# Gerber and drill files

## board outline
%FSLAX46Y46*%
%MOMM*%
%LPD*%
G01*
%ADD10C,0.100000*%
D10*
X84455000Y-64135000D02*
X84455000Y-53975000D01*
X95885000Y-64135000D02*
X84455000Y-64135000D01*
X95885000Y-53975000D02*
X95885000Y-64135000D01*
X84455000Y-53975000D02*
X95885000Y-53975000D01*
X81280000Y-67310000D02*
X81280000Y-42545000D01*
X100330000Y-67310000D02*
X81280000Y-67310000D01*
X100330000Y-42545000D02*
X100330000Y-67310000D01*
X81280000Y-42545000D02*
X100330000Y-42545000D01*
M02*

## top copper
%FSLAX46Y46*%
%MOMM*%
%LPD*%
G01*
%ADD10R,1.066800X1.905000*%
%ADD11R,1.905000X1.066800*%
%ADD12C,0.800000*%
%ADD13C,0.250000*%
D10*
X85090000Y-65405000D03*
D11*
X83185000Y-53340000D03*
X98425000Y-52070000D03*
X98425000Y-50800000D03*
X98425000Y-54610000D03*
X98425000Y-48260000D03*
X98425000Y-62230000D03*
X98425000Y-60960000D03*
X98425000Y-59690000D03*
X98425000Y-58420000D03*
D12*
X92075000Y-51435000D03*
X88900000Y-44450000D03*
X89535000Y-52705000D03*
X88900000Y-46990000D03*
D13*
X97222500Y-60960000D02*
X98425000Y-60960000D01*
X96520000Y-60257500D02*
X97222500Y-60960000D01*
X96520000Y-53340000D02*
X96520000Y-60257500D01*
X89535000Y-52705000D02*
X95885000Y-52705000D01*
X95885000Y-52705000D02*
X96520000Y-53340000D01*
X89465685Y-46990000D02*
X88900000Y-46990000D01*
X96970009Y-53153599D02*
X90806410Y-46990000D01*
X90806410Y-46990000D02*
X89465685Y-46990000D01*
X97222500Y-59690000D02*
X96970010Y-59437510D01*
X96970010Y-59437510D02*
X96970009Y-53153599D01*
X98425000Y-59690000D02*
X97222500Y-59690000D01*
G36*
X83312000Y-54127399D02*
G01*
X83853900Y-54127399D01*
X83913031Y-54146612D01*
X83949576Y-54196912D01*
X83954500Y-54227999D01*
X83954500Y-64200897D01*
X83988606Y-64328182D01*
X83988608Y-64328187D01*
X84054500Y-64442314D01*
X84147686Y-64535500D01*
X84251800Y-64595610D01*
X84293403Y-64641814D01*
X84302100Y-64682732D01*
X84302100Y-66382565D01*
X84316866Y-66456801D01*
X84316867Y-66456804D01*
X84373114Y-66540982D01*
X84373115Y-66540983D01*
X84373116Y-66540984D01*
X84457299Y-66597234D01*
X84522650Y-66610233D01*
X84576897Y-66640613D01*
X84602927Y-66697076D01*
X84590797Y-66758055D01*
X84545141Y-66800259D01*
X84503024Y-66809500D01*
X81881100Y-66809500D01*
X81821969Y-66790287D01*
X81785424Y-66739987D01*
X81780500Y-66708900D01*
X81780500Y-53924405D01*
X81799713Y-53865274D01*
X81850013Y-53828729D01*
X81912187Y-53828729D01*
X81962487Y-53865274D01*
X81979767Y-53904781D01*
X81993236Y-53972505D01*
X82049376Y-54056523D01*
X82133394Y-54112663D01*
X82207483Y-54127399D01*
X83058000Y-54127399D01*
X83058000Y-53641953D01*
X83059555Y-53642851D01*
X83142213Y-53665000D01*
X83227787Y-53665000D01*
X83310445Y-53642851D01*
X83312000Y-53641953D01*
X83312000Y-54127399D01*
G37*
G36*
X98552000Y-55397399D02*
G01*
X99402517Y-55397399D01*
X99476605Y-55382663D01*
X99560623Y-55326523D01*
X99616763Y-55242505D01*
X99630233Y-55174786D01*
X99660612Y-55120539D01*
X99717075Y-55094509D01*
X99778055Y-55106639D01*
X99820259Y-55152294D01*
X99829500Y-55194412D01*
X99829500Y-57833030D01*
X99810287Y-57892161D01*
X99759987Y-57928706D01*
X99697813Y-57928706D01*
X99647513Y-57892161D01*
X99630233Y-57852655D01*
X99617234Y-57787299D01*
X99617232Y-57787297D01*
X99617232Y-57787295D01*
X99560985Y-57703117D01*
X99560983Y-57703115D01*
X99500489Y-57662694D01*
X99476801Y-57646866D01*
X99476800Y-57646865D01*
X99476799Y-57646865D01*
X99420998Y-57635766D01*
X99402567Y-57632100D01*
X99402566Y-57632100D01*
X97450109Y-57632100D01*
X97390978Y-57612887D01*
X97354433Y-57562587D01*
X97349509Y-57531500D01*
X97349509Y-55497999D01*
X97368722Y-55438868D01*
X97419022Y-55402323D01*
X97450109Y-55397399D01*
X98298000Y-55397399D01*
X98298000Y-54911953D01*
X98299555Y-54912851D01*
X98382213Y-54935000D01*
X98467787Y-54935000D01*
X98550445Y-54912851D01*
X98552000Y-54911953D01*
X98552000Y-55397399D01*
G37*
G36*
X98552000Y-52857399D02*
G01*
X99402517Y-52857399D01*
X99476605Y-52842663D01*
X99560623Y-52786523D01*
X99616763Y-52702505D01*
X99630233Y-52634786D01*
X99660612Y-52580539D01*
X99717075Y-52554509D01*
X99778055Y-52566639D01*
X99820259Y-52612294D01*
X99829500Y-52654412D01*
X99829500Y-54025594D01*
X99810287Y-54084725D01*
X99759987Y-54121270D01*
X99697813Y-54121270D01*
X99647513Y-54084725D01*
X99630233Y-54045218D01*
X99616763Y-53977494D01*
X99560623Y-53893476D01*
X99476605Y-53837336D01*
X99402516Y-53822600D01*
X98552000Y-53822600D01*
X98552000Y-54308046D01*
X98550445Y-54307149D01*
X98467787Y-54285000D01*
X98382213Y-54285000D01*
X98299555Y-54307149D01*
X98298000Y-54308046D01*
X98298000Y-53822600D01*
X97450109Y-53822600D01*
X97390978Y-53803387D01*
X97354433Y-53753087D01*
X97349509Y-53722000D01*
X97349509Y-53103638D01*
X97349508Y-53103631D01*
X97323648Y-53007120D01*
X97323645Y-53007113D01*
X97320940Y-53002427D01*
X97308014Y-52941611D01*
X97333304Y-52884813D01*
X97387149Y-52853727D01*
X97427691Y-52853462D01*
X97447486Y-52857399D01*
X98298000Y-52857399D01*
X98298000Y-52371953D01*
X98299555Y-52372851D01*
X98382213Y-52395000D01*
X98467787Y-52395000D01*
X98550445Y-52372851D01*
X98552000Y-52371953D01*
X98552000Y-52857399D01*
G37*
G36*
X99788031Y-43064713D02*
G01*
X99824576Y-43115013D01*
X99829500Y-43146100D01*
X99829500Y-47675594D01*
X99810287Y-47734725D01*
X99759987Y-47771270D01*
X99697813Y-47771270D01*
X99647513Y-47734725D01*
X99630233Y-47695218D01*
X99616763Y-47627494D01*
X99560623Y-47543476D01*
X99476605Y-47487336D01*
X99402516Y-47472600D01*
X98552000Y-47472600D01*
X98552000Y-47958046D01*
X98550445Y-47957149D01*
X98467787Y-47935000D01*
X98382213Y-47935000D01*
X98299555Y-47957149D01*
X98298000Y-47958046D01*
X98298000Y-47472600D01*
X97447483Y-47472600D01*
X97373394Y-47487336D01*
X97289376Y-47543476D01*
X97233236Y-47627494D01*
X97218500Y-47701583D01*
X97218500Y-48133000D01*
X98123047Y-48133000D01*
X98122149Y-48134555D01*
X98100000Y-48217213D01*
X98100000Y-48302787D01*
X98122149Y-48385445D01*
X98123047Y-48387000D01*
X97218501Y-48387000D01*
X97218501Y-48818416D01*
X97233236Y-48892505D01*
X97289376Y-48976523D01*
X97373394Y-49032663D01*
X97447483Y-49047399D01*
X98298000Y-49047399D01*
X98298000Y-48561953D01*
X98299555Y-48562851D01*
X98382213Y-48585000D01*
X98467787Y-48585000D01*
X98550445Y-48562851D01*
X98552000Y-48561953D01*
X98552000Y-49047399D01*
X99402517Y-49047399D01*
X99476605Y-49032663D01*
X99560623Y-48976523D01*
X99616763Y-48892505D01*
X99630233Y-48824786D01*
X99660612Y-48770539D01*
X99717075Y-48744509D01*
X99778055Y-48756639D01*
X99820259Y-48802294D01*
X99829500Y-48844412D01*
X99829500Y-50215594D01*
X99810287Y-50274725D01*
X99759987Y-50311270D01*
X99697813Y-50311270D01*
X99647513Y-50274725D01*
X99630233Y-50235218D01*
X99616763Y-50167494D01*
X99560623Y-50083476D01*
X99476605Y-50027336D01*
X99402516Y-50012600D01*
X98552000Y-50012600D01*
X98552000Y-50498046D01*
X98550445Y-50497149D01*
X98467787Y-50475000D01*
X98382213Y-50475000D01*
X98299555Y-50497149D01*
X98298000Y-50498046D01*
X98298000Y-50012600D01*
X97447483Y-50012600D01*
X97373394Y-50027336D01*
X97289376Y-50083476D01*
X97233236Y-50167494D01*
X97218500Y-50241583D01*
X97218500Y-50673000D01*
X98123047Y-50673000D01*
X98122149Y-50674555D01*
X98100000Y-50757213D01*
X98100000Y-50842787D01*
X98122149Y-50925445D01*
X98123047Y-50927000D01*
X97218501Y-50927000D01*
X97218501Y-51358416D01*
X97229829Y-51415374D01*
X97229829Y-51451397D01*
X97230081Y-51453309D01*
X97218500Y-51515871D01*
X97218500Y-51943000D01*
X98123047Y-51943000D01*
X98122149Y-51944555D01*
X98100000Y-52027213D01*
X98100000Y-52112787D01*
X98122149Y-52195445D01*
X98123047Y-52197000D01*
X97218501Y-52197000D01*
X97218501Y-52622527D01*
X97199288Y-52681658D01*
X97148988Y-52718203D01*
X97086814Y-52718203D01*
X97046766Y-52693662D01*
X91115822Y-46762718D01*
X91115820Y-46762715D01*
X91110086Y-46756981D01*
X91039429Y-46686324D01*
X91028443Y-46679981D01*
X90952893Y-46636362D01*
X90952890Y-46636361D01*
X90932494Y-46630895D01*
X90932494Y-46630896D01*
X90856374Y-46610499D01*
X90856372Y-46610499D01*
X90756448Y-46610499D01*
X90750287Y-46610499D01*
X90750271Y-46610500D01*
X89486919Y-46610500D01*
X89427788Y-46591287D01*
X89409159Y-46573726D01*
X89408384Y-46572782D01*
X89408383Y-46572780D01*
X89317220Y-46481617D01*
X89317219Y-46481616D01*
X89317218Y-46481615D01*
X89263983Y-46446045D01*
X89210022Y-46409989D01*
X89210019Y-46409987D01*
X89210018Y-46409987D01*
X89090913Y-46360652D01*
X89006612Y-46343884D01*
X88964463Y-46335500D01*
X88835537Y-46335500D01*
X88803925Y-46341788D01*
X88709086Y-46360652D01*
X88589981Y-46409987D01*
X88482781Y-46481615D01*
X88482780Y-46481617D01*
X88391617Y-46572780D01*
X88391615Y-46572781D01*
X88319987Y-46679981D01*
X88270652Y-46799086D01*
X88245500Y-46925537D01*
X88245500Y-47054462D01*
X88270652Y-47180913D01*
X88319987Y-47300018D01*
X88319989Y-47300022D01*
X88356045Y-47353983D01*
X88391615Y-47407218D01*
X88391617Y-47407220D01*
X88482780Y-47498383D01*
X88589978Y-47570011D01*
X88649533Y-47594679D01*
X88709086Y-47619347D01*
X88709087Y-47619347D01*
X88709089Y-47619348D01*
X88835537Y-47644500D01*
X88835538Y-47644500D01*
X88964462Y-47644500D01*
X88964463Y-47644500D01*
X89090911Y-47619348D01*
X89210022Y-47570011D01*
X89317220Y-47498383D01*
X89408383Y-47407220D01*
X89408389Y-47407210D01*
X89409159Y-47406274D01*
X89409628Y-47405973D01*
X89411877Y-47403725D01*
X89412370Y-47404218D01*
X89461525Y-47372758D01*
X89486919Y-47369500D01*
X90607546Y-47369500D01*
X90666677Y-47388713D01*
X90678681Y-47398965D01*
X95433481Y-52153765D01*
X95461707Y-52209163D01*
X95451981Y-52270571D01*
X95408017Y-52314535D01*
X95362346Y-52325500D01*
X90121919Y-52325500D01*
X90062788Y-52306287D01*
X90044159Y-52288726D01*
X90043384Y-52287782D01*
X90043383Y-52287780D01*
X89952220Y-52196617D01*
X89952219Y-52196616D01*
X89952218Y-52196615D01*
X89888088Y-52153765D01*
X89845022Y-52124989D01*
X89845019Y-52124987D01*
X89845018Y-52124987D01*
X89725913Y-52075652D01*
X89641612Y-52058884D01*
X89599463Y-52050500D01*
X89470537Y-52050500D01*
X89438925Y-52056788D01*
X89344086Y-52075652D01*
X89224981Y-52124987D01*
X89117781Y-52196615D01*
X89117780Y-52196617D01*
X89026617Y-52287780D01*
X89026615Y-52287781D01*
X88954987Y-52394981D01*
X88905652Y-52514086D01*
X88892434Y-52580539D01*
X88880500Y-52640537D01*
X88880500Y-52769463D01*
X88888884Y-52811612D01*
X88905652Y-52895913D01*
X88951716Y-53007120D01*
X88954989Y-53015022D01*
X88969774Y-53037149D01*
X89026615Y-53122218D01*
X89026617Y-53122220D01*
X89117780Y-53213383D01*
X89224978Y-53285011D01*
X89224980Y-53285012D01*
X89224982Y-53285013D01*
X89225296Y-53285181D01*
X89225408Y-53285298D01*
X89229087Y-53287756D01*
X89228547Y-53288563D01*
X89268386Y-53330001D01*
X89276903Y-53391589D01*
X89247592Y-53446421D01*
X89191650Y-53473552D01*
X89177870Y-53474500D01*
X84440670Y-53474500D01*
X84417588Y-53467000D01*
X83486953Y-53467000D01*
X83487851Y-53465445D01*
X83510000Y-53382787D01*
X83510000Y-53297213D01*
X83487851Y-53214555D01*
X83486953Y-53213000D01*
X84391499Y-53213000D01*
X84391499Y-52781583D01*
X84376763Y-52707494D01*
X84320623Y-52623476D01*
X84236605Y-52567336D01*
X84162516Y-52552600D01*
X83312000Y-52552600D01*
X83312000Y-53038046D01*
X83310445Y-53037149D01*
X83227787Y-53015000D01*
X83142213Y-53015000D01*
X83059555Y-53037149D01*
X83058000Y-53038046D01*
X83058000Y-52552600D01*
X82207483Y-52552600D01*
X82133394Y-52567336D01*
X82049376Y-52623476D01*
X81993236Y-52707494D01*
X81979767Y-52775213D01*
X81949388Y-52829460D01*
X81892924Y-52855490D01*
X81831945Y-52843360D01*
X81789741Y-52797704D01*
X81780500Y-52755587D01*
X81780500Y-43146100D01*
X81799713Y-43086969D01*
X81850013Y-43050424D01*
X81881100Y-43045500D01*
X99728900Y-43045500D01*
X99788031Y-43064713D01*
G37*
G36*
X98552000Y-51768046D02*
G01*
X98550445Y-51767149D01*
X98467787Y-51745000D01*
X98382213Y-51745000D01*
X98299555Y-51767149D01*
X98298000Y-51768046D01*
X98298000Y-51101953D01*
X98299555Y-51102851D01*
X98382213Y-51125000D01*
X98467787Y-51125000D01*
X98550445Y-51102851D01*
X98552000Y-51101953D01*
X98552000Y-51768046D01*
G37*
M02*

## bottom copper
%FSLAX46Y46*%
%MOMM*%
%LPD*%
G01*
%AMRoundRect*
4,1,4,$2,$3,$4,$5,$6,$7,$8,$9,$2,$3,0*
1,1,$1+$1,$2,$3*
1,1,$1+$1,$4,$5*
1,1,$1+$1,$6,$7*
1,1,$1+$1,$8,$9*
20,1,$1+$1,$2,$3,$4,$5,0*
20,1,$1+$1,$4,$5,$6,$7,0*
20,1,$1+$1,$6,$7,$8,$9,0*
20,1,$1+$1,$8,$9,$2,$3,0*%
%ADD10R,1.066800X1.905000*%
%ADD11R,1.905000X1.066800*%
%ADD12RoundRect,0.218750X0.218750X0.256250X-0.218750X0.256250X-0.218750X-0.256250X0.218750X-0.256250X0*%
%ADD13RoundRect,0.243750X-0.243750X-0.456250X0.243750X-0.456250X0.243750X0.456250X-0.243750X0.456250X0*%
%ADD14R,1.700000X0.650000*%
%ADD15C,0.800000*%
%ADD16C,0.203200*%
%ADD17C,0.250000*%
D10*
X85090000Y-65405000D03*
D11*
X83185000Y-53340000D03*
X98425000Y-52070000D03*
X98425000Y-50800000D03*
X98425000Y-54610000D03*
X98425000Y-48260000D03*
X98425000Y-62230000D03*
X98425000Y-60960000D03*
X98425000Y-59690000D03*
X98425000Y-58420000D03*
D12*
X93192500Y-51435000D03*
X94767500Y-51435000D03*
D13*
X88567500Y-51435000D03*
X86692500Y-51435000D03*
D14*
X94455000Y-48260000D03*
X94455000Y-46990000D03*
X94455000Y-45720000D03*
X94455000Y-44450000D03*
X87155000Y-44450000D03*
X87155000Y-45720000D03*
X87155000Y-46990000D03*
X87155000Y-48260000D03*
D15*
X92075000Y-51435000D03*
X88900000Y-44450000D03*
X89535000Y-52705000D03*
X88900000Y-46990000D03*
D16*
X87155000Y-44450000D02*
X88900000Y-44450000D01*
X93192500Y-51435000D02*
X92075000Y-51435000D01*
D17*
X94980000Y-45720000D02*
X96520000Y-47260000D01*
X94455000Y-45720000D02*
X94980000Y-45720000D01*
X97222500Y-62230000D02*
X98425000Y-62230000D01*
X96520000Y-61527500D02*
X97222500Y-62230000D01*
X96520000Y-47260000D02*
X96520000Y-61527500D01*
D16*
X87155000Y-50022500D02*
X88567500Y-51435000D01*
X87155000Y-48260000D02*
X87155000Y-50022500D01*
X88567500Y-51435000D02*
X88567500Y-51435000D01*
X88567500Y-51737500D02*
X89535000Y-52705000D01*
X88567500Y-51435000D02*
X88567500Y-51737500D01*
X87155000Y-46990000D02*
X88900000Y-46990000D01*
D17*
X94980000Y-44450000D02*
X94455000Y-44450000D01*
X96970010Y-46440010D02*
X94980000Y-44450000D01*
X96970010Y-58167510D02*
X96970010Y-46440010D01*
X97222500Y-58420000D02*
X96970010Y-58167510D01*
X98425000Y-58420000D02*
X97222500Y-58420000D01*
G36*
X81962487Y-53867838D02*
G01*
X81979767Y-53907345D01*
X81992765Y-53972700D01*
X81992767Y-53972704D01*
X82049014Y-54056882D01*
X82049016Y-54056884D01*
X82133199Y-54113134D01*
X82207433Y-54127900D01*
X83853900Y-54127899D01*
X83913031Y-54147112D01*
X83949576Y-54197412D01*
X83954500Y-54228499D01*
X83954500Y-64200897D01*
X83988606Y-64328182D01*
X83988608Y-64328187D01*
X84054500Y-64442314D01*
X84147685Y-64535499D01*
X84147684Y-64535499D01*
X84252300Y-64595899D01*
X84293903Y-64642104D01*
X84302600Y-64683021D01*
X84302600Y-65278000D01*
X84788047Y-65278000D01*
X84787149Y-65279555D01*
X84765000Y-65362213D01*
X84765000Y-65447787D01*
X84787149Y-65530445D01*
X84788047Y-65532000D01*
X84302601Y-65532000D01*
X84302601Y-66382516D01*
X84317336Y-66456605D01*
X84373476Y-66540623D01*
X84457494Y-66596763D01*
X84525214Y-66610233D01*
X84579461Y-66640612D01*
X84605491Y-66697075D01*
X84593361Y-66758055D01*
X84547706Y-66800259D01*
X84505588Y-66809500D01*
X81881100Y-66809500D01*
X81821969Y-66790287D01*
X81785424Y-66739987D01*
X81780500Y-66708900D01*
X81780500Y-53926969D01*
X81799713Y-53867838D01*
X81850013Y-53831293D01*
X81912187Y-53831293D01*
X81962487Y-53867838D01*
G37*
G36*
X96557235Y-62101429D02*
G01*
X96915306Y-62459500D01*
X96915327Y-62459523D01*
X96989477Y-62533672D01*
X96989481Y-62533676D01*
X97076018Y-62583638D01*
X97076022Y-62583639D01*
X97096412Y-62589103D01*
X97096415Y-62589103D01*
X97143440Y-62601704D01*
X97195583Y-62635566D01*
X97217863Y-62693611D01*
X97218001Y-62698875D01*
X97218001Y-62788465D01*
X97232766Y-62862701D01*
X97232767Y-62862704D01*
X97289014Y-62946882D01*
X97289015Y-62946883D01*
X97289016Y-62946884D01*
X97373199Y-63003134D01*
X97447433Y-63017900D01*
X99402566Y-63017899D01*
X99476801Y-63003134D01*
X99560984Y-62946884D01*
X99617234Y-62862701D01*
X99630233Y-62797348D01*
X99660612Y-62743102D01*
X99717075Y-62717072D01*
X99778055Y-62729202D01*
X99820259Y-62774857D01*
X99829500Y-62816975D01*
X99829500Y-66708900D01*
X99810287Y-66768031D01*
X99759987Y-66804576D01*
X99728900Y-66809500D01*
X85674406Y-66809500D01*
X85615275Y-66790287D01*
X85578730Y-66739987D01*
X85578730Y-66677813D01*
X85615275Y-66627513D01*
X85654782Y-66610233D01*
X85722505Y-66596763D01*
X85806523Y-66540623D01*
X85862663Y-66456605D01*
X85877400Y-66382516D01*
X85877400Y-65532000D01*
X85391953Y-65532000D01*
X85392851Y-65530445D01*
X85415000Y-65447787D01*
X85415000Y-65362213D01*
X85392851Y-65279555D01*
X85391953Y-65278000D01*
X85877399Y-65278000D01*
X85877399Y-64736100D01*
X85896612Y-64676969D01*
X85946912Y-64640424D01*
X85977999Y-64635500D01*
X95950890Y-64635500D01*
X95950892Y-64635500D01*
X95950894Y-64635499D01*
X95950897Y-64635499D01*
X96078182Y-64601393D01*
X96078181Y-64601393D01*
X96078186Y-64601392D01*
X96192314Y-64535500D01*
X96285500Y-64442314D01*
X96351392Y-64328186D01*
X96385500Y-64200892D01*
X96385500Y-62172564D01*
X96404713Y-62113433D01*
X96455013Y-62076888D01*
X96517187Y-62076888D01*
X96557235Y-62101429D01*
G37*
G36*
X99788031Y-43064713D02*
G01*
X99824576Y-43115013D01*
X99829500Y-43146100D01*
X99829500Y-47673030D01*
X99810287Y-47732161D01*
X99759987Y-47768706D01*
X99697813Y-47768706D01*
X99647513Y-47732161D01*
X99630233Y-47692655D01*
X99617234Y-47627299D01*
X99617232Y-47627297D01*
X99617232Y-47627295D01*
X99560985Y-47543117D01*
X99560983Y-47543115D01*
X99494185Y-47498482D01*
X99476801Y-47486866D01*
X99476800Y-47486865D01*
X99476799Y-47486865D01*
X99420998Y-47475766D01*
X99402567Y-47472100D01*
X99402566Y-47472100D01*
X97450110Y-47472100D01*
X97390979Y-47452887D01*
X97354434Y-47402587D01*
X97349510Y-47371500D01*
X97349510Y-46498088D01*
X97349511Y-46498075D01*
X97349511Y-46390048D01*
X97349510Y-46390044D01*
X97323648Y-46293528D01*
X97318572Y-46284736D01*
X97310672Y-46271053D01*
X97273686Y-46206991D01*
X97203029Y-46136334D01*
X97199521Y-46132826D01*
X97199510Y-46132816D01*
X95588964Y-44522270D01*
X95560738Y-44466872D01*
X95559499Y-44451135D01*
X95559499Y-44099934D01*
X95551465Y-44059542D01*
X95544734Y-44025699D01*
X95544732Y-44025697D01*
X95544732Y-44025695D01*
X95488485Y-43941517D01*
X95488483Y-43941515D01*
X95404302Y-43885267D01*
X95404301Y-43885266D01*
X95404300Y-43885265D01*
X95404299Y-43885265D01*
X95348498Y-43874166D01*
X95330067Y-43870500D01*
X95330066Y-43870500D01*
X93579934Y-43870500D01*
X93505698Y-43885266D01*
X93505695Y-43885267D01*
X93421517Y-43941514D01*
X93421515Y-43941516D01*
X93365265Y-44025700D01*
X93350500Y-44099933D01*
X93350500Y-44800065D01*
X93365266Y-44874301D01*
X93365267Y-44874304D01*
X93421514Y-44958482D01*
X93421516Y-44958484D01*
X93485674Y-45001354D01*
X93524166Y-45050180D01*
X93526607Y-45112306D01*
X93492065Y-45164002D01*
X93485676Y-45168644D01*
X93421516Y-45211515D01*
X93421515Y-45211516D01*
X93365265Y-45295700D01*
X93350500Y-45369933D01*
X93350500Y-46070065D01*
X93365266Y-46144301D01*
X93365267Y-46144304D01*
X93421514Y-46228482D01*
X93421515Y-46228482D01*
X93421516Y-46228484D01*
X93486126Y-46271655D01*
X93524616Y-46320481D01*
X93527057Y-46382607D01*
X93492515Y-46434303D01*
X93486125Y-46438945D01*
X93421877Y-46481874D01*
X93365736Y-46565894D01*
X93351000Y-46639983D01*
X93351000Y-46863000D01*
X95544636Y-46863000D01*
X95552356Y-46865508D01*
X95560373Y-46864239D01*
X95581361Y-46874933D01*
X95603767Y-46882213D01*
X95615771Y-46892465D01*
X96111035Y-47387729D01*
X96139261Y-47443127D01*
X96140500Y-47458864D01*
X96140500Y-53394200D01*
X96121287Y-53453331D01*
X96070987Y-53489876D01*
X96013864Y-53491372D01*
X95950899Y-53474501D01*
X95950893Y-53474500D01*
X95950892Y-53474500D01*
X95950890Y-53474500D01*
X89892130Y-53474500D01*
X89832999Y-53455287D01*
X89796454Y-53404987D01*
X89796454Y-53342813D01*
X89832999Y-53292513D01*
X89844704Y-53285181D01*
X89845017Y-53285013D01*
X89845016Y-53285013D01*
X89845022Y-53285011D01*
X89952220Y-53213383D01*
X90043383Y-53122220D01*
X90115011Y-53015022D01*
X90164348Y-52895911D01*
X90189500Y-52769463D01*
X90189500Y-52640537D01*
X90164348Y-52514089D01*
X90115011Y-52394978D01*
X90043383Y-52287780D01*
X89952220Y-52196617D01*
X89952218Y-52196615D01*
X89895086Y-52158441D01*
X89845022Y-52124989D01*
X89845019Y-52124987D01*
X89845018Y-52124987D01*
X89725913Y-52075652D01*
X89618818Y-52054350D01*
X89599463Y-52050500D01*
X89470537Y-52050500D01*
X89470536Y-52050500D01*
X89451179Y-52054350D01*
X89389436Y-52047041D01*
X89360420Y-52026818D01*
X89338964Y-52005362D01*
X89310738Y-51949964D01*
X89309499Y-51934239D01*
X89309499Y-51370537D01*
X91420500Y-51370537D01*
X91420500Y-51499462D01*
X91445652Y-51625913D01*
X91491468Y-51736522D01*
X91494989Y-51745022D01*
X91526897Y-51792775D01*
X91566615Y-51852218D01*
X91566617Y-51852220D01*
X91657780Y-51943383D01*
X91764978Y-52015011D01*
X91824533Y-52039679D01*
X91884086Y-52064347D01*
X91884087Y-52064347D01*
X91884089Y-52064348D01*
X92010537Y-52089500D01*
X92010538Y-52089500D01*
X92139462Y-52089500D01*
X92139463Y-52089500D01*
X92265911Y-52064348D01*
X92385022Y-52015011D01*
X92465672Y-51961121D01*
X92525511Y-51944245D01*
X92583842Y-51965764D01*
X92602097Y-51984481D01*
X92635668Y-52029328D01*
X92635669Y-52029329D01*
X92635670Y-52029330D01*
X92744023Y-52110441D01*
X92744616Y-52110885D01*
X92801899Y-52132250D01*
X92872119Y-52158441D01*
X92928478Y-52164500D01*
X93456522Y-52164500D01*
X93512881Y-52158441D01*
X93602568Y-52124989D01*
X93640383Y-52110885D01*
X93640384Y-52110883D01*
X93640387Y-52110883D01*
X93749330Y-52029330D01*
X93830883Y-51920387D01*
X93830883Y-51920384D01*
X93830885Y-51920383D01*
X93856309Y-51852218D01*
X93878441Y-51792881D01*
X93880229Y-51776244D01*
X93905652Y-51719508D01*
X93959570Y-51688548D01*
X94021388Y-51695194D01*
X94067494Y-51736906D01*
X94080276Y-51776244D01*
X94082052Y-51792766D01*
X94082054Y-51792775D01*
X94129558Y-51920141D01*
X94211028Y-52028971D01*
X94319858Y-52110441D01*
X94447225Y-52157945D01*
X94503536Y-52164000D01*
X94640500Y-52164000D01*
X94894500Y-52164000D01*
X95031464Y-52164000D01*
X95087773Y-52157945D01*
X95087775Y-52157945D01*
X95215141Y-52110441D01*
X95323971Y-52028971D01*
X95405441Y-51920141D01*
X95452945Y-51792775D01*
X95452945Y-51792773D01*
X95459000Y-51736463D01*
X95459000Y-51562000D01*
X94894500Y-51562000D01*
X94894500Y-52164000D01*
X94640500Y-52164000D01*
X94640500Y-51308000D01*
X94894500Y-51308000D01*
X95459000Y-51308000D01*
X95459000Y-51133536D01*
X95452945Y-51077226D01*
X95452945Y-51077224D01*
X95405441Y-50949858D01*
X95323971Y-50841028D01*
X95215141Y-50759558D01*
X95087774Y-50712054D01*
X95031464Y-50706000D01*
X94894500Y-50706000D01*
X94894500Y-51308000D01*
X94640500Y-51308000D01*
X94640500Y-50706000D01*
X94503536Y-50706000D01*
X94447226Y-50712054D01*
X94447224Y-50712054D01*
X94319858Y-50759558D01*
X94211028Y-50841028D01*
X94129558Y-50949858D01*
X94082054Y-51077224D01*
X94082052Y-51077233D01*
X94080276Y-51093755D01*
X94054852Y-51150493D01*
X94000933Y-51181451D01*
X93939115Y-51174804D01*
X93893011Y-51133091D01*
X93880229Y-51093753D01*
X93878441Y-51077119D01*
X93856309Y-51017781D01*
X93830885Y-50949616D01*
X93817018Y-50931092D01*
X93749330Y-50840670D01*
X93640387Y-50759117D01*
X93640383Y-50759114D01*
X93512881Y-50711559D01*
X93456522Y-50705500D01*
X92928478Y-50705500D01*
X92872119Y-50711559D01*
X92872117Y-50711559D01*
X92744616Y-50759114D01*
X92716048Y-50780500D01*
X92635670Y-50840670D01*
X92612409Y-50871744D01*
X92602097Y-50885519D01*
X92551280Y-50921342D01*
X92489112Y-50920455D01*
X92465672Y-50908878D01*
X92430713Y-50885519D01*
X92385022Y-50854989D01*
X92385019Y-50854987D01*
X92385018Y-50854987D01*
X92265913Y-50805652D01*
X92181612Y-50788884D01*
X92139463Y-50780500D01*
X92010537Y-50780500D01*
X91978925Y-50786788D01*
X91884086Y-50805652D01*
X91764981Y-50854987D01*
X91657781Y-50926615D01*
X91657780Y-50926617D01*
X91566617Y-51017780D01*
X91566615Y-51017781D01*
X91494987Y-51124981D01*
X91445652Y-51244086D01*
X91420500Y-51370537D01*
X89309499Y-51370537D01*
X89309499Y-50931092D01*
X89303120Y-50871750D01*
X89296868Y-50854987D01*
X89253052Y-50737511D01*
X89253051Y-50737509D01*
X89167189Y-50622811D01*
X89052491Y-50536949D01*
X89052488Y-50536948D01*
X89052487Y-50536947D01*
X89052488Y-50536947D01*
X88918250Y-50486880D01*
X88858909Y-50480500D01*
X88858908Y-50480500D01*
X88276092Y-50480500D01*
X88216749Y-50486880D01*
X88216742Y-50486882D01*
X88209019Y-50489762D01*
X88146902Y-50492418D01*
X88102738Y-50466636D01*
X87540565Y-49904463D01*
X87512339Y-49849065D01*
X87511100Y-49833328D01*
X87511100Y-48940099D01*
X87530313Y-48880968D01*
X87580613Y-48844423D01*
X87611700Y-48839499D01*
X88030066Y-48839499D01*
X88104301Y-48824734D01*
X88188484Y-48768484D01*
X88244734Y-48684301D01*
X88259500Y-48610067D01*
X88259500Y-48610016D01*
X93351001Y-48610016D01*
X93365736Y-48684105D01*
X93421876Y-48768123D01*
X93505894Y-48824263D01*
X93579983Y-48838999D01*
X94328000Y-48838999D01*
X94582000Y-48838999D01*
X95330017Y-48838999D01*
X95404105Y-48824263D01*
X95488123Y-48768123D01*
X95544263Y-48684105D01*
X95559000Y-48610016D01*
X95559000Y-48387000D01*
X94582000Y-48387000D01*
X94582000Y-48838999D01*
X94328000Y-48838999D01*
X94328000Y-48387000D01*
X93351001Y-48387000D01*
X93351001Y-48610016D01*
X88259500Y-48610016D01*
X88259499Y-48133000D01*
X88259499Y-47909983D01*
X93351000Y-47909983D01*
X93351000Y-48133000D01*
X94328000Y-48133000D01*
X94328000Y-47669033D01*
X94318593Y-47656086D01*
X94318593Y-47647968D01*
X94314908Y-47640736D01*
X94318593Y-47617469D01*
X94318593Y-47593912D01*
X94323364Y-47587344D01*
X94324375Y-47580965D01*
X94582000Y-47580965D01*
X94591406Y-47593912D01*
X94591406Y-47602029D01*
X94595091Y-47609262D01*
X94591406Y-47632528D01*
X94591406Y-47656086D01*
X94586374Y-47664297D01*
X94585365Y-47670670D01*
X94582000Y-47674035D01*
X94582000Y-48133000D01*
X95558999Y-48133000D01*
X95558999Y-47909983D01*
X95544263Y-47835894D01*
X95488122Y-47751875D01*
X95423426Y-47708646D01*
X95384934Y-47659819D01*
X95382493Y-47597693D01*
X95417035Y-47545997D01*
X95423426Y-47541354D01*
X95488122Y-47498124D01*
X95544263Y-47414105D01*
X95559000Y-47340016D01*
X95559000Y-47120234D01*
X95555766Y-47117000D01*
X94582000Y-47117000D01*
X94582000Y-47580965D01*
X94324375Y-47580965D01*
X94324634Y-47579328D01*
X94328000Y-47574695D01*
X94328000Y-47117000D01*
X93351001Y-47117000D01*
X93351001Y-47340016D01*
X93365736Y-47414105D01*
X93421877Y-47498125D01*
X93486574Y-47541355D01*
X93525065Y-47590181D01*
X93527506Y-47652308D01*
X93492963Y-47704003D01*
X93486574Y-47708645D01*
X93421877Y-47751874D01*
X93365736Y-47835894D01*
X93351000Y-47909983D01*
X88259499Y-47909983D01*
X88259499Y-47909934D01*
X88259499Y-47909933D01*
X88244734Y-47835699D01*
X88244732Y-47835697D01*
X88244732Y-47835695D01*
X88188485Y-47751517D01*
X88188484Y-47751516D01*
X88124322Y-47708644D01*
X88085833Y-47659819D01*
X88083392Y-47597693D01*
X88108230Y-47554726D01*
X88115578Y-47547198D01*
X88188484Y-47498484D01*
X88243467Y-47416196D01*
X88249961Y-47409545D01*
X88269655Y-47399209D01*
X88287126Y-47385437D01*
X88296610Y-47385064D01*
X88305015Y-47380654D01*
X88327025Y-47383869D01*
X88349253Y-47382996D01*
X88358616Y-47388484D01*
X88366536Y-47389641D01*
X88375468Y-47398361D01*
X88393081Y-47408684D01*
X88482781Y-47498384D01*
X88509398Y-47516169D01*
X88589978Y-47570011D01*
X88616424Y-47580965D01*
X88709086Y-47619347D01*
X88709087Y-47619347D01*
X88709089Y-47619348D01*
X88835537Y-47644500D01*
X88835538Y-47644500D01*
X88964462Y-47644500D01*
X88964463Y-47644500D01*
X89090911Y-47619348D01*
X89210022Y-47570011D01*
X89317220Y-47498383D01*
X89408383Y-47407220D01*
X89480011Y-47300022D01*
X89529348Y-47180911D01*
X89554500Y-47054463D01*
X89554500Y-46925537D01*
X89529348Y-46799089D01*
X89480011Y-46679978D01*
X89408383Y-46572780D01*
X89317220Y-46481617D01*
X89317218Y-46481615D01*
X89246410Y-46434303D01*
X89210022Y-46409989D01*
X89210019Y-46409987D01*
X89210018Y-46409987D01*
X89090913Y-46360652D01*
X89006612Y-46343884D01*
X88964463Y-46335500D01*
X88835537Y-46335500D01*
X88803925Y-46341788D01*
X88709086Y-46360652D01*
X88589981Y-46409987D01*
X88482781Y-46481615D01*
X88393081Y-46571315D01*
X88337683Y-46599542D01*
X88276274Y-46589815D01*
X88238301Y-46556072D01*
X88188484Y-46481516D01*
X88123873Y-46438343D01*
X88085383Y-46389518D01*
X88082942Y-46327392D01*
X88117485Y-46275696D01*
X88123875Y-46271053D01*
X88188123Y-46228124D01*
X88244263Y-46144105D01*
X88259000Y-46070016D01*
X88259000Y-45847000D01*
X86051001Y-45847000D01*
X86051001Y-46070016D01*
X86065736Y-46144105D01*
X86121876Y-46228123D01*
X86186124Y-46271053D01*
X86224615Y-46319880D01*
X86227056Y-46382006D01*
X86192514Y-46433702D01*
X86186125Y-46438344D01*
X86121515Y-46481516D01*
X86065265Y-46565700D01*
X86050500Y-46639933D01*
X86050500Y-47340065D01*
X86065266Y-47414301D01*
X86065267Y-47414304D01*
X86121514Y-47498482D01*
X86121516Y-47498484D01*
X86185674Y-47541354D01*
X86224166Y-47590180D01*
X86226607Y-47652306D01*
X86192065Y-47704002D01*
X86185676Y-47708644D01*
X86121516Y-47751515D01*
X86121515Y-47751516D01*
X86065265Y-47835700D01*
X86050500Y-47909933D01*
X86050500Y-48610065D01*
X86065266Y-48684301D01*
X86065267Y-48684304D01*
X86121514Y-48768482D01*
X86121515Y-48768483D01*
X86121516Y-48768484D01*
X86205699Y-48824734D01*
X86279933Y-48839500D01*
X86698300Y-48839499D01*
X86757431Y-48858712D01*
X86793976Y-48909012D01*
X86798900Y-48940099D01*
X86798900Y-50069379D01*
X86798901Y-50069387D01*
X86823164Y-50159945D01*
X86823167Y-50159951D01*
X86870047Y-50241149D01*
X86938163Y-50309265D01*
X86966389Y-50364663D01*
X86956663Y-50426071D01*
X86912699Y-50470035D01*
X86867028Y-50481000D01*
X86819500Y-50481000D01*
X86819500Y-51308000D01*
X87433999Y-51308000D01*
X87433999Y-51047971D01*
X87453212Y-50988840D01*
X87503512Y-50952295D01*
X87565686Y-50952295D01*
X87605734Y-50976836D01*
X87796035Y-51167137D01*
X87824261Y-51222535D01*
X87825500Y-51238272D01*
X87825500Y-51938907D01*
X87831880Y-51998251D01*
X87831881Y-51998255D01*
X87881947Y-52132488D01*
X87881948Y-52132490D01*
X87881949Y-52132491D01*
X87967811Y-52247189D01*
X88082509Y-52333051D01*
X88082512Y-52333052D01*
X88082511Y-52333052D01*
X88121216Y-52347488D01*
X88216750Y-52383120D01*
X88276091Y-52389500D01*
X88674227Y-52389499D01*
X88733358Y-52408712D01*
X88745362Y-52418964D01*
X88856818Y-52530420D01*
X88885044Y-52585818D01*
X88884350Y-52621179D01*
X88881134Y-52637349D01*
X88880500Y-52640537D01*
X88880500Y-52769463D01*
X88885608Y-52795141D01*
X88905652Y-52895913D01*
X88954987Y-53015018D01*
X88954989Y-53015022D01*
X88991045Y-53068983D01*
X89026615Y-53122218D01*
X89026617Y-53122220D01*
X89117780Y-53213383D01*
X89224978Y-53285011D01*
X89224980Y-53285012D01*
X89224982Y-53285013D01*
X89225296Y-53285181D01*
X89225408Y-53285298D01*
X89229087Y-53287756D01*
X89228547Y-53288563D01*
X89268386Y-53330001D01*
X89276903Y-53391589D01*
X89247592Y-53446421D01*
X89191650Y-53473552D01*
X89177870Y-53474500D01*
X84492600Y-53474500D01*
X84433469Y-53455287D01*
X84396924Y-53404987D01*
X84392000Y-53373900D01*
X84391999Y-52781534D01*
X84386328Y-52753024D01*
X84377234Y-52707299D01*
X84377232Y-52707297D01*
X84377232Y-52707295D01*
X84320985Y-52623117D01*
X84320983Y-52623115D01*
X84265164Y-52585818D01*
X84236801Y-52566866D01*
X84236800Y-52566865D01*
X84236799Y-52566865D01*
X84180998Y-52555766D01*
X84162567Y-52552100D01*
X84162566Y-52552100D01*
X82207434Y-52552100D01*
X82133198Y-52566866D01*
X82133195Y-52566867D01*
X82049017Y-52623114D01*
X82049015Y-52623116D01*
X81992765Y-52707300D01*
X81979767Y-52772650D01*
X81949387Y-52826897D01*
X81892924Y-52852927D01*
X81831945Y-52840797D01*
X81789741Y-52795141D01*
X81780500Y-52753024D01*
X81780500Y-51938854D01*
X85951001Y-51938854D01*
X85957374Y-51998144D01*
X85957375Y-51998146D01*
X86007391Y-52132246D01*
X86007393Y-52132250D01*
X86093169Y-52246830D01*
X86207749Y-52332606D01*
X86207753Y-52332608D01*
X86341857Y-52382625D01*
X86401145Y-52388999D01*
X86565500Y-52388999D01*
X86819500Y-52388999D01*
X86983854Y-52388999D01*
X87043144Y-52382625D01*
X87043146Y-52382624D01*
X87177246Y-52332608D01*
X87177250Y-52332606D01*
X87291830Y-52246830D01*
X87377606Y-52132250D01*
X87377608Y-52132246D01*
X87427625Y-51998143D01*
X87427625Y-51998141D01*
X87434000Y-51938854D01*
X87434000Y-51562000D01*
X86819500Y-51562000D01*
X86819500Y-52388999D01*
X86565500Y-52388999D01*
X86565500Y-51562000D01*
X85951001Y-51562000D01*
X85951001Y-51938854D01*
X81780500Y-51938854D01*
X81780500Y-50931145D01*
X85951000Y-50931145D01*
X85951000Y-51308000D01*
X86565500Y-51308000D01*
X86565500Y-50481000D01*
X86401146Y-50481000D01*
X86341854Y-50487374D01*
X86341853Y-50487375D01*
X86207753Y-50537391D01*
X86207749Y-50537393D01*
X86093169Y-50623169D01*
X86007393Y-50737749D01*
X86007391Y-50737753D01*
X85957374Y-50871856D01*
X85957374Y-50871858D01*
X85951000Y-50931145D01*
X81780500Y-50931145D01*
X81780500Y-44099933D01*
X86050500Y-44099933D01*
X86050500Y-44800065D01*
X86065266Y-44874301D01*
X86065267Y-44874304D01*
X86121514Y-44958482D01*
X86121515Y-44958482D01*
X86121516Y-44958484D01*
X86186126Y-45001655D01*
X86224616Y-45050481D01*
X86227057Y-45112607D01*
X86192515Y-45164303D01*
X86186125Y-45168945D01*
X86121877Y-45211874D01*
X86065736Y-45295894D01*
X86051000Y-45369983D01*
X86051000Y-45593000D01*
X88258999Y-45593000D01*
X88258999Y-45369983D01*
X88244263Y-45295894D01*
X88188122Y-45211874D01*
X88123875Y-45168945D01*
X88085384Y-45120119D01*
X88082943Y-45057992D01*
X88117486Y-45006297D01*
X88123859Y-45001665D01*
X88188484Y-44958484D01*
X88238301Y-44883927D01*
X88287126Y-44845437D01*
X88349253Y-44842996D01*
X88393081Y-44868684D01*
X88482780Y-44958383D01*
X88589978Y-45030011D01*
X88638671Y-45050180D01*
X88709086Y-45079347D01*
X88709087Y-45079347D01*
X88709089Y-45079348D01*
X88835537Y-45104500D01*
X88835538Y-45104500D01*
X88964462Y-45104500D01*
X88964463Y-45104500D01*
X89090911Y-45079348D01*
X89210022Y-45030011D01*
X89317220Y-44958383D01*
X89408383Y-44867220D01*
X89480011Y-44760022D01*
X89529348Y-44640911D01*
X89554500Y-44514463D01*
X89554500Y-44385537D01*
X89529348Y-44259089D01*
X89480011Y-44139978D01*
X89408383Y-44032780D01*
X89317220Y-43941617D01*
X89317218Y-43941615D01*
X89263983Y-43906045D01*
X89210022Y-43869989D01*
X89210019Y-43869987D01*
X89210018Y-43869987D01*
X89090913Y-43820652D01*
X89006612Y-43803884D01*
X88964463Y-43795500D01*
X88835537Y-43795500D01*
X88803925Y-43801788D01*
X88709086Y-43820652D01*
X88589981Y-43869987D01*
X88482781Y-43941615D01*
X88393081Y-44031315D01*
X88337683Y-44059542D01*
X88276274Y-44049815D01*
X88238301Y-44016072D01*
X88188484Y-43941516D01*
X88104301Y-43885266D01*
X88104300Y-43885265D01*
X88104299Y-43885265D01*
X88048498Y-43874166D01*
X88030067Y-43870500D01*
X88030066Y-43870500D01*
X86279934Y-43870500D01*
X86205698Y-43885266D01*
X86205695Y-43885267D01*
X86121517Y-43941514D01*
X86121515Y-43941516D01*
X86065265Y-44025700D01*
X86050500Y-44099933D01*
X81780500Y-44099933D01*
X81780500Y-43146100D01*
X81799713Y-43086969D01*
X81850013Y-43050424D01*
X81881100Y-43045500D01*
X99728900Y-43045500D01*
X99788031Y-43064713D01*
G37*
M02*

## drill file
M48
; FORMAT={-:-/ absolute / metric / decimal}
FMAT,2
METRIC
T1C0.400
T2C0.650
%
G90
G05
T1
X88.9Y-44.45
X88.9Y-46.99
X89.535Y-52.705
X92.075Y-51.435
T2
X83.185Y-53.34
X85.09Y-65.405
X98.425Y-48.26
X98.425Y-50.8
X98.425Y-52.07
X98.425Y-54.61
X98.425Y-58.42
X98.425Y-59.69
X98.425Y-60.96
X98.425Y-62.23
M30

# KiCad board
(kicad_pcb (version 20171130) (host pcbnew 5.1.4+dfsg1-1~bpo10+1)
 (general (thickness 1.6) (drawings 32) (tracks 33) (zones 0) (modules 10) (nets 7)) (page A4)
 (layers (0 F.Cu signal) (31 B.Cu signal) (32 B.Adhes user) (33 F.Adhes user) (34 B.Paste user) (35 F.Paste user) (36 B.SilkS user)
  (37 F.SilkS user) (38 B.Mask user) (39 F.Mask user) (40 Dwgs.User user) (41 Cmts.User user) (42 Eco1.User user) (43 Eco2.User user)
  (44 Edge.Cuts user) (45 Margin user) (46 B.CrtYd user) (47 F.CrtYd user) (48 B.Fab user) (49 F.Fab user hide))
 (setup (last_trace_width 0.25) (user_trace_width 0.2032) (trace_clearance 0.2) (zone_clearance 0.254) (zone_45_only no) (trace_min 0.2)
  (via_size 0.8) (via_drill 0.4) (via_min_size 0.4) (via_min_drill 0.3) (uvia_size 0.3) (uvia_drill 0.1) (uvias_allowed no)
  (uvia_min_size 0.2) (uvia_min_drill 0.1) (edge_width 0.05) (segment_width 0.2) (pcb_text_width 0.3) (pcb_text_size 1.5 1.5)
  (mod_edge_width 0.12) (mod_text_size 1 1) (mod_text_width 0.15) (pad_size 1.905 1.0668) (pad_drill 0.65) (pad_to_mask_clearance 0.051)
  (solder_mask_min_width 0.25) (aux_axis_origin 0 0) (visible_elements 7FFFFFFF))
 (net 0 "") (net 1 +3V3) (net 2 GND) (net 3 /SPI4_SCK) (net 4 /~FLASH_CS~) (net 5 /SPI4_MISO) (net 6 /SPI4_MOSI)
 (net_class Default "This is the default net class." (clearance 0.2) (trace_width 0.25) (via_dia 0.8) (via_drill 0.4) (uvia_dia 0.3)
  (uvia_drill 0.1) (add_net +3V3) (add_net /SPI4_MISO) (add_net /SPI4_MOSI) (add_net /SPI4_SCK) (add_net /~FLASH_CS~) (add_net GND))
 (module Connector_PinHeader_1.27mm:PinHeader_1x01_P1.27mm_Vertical (layer F.Cu) (at 85.09 65.405 90)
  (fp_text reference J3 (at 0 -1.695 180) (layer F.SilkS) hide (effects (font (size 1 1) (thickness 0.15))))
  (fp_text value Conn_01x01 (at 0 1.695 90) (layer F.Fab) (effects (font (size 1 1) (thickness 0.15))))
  (pad 1 thru_hole rect (at 0 0 90) (size 1.905 1.0668) (drill 0.65) (layers *.Cu *.Mask) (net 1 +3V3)))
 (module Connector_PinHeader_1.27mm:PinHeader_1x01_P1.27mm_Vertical (layer F.Cu) (at 83.185 53.34)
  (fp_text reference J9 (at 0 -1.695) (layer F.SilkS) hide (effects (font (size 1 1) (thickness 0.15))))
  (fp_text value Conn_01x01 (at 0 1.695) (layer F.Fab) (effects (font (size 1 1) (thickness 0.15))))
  (pad 1 thru_hole rect (at 0 0) (size 1.905 1.0668) (drill 0.65) (layers *.Cu *.Mask) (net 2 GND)))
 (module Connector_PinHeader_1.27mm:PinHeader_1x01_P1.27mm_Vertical (layer F.Cu) (at 98.425 52.07)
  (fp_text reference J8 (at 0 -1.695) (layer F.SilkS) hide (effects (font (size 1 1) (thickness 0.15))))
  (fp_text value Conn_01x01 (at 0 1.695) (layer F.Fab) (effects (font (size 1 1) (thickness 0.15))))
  (pad 1 thru_hole rect (at 0 0) (size 1.905 1.0668) (drill 0.65) (layers *.Cu *.Mask) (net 2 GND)))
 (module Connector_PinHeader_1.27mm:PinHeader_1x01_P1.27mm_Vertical (layer F.Cu) (at 98.425 50.8)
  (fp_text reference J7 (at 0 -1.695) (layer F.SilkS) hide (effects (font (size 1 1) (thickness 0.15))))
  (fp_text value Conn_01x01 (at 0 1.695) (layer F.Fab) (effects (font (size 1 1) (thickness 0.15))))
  (pad 1 thru_hole rect (at 0 0) (size 1.905 1.0668) (drill 0.65) (layers *.Cu *.Mask) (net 2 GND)))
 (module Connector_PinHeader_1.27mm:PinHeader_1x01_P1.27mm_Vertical (layer F.Cu) (at 98.425 54.61)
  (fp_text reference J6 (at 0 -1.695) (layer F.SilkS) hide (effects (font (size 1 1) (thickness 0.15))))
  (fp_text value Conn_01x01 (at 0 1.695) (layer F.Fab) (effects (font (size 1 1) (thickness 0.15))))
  (pad 1 thru_hole rect (at 0 0) (size 1.905 1.0668) (drill 0.65) (layers *.Cu *.Mask) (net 2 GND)))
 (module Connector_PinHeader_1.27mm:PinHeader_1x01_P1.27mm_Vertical (layer F.Cu) (at 98.425 48.26)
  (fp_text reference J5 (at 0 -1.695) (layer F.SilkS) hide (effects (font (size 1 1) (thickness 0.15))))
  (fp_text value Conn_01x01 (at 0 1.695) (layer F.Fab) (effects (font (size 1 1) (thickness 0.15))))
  (pad 1 thru_hole rect (at 0 0) (size 1.905 1.0668) (drill 0.65) (layers *.Cu *.Mask) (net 2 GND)))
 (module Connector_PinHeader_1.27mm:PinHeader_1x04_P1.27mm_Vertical (layer F.Cu) (at 98.425 58.42)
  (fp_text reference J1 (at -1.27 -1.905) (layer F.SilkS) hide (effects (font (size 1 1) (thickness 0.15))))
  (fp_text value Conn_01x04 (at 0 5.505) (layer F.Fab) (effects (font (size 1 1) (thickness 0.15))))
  (pad 4 thru_hole rect (at 0 3.81) (size 1.905 1.0668) (drill 0.65) (layers *.Cu *.Mask) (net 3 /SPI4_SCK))
  (pad 3 thru_hole rect (at 0 2.54) (size 1.905 1.0668) (drill 0.65) (layers *.Cu *.Mask) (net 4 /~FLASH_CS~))
  (pad 2 thru_hole rect (at 0 1.27) (size 1.905 1.0668) (drill 0.65) (layers *.Cu *.Mask) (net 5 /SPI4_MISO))
  (pad 1 thru_hole rect (at 0 0) (size 1.905 1.0668) (drill 0.65) (layers *.Cu *.Mask) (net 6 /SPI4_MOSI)))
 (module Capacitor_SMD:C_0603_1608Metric (layer B.Cu) (at 93.98 51.435 180)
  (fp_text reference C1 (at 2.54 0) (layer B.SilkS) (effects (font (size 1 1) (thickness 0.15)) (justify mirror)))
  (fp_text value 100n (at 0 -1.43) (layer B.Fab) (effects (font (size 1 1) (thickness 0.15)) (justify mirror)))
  (pad 2 smd roundrect (at 0.7875 0 180) (size 0.875 0.95) (layers B.Cu B.Paste B.Mask) (roundrect_rratio 0.25) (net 2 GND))
  (pad 1 smd roundrect (at -0.7875 0 180) (size 0.875 0.95) (layers B.Cu B.Paste B.Mask) (roundrect_rratio 0.25) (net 1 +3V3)))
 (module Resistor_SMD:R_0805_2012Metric (layer B.Cu) (at 87.63 51.435)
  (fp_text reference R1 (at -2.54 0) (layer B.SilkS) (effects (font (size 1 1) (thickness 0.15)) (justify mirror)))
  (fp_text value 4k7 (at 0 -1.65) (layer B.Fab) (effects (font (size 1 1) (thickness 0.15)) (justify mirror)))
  (pad 2 smd roundrect (at 0.9375 0) (size 0.975 1.4) (layers B.Cu B.Paste B.Mask) (roundrect_rratio 0.25) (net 4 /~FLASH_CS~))
  (pad 1 smd roundrect (at -0.9375 0) (size 0.975 1.4) (layers B.Cu B.Paste B.Mask) (roundrect_rratio 0.25) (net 1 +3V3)))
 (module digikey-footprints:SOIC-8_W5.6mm (layer B.Cu) (at 90.805 46.355 90)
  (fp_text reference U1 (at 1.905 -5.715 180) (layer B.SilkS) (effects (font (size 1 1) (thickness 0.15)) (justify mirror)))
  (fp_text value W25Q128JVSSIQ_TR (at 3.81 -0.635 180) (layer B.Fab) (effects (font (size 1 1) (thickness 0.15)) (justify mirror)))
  (pad 8 smd rect (at -1.905 3.65 90) (size 0.65 1.7) (layers B.Cu B.Paste B.Mask) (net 1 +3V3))
  (pad 7 smd rect (at -0.635 3.65 90) (size 0.65 1.7) (layers B.Cu B.Paste B.Mask) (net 1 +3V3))
  (pad 6 smd rect (at 0.635 3.65 90) (size 0.65 1.7) (layers B.Cu B.Paste B.Mask) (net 3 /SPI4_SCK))
  (pad 5 smd rect (at 1.905 3.65 90) (size 0.65 1.7) (layers B.Cu B.Paste B.Mask) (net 6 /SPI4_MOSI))
  (pad 4 smd rect (at 1.905 -3.65 90) (size 0.65 1.7) (layers B.Cu B.Paste B.Mask) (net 2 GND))
  (pad 3 smd rect (at 0.635 -3.65 90) (size 0.65 1.7) (layers B.Cu B.Paste B.Mask) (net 1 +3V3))
  (pad 2 smd rect (at -0.635 -3.65 90) (size 0.65 1.7) (layers B.Cu B.Paste B.Mask) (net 5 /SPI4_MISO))
  (pad 1 smd rect (at -1.905 -3.65 90) (size 0.65 1.7) (layers B.Cu B.Paste B.Mask) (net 4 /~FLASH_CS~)))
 (gr_line (start 84.455 64.135) (end 84.455 53.975) (layer Edge.Cuts) (width 0.1))
 (gr_line (start 95.885 64.135) (end 84.455 64.135) (layer Edge.Cuts) (width 0.1))
 (gr_line (start 95.885 53.975) (end 95.885 64.135) (layer Edge.Cuts) (width 0.1))
 (gr_line (start 84.455 53.975) (end 95.885 53.975) (layer Edge.Cuts) (width 0.1))
 (gr_line (start 81.28 67.31) (end 81.28 42.545) (layer Edge.Cuts) (width 0.1))
 (gr_line (start 100.33 67.31) (end 81.28 67.31) (layer Edge.Cuts) (width 0.1))
 (gr_line (start 100.33 42.545) (end 100.33 67.31) (layer Edge.Cuts) (width 0.1))
 (gr_line (start 81.28 42.545) (end 100.33 42.545) (layer Edge.Cuts) (width 0.1))
 (via (at 92.075 51.435) (size 0.8) (drill 0.4) (layers F.Cu B.Cu) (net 2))
 (via (at 88.9 44.45) (size 0.8) (drill 0.4) (layers F.Cu B.Cu) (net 2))
 (segment (start 87.155 44.45) (end 88.9 44.45) (width 0.2032) (layer B.Cu) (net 2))
 (segment (start 93.1925 51.435) (end 92.075 51.435) (width 0.2032) (layer B.Cu) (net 2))
 (segment (start 94.98 45.72) (end 96.52 47.26) (width 0.25) (layer B.Cu) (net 3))
 (segment (start 94.455 45.72) (end 94.98 45.72) (width 0.25) (layer B.Cu) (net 3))
 (segment (start 97.2225 62.23) (end 98.425 62.23) (width 0.25) (layer B.Cu) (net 3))
 (segment (start 96.52 61.5275) (end 97.2225 62.23) (width 0.25) (layer B.Cu) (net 3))
 (segment (start 96.52 47.26) (end 96.52 61.5275) (width 0.25) (layer B.Cu) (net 3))
 (segment (start 87.155 50.0225) (end 88.5675 51.435) (width 0.2032) (layer B.Cu) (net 4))
 (segment (start 87.155 48.26) (end 87.155 50.0225) (width 0.2032) (layer B.Cu) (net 4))
 (segment (start 88.5675 51.435) (end 88.5675 51.435) (width 0.2032) (layer B.Cu) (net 4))
 (via (at 89.535 52.705) (size 0.8) (drill 0.4) (layers F.Cu B.Cu) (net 4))
 (segment (start 88.5675 51.7375) (end 89.535 52.705) (width 0.2032) (layer B.Cu) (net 4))
 (segment (start 88.5675 51.435) (end 88.5675 51.7375) (width 0.2032) (layer B.Cu) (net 4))
 (segment (start 97.2225 60.96) (end 98.425 60.96) (width 0.25) (layer F.Cu) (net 4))
 (segment (start 96.52 60.2575) (end 97.2225 60.96) (width 0.25) (layer F.Cu) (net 4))
 (segment (start 96.52 53.34) (end 96.52 60.2575) (width 0.25) (layer F.Cu) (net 4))
 (segment (start 89.535 52.705) (end 95.885 52.705) (width 0.25) (layer F.Cu) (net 4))
 (segment (start 95.885 52.705) (end 96.52 53.34) (width 0.25) (layer F.Cu) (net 4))
 (via (at 88.9 46.99) (size 0.8) (drill 0.4) (layers F.Cu B.Cu) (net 5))
 (segment (start 87.155 46.99) (end 88.9 46.99) (width 0.2032) (layer B.Cu) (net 5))
 (segment (start 89.465685 46.99) (end 88.9 46.99) (width 0.25) (layer F.Cu) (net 5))
 (segment (start 96.970009 53.153599) (end 90.80641 46.99) (width 0.25) (layer F.Cu) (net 5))
 (segment (start 90.80641 46.99) (end 89.465685 46.99) (width 0.25) (layer F.Cu) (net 5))
 (segment (start 97.2225 59.69) (end 96.97001 59.43751) (width 0.25) (layer F.Cu) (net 5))
 (segment (start 96.97001 59.43751) (end 96.970009 53.153599) (width 0.25) (layer F.Cu) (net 5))
 (segment (start 98.425 59.69) (end 97.2225 59.69) (width 0.25) (layer F.Cu) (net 5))
 (segment (start 94.98 44.45) (end 94.455 44.45) (width 0.25) (layer B.Cu) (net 6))
 (segment (start 96.97001 46.44001) (end 94.98 44.45) (width 0.25) (layer B.Cu) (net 6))
 (segment (start 96.97001 58.16751) (end 96.97001 46.44001) (width 0.25) (layer B.Cu) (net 6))
 (segment (start 97.2225 58.42) (end 96.97001 58.16751) (width 0.25) (layer B.Cu) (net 6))
 (segment (start 98.425 58.42) (end 97.2225 58.42) (width 0.25) (layer B.Cu) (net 6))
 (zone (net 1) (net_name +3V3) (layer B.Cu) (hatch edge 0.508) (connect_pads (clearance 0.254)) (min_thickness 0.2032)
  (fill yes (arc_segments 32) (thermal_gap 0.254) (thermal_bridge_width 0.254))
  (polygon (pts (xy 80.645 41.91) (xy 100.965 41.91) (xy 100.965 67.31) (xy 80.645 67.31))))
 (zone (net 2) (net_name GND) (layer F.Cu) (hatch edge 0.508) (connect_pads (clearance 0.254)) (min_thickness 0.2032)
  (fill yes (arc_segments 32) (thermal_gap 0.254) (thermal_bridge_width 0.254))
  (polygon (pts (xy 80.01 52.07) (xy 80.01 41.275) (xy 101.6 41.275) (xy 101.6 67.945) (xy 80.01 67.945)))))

